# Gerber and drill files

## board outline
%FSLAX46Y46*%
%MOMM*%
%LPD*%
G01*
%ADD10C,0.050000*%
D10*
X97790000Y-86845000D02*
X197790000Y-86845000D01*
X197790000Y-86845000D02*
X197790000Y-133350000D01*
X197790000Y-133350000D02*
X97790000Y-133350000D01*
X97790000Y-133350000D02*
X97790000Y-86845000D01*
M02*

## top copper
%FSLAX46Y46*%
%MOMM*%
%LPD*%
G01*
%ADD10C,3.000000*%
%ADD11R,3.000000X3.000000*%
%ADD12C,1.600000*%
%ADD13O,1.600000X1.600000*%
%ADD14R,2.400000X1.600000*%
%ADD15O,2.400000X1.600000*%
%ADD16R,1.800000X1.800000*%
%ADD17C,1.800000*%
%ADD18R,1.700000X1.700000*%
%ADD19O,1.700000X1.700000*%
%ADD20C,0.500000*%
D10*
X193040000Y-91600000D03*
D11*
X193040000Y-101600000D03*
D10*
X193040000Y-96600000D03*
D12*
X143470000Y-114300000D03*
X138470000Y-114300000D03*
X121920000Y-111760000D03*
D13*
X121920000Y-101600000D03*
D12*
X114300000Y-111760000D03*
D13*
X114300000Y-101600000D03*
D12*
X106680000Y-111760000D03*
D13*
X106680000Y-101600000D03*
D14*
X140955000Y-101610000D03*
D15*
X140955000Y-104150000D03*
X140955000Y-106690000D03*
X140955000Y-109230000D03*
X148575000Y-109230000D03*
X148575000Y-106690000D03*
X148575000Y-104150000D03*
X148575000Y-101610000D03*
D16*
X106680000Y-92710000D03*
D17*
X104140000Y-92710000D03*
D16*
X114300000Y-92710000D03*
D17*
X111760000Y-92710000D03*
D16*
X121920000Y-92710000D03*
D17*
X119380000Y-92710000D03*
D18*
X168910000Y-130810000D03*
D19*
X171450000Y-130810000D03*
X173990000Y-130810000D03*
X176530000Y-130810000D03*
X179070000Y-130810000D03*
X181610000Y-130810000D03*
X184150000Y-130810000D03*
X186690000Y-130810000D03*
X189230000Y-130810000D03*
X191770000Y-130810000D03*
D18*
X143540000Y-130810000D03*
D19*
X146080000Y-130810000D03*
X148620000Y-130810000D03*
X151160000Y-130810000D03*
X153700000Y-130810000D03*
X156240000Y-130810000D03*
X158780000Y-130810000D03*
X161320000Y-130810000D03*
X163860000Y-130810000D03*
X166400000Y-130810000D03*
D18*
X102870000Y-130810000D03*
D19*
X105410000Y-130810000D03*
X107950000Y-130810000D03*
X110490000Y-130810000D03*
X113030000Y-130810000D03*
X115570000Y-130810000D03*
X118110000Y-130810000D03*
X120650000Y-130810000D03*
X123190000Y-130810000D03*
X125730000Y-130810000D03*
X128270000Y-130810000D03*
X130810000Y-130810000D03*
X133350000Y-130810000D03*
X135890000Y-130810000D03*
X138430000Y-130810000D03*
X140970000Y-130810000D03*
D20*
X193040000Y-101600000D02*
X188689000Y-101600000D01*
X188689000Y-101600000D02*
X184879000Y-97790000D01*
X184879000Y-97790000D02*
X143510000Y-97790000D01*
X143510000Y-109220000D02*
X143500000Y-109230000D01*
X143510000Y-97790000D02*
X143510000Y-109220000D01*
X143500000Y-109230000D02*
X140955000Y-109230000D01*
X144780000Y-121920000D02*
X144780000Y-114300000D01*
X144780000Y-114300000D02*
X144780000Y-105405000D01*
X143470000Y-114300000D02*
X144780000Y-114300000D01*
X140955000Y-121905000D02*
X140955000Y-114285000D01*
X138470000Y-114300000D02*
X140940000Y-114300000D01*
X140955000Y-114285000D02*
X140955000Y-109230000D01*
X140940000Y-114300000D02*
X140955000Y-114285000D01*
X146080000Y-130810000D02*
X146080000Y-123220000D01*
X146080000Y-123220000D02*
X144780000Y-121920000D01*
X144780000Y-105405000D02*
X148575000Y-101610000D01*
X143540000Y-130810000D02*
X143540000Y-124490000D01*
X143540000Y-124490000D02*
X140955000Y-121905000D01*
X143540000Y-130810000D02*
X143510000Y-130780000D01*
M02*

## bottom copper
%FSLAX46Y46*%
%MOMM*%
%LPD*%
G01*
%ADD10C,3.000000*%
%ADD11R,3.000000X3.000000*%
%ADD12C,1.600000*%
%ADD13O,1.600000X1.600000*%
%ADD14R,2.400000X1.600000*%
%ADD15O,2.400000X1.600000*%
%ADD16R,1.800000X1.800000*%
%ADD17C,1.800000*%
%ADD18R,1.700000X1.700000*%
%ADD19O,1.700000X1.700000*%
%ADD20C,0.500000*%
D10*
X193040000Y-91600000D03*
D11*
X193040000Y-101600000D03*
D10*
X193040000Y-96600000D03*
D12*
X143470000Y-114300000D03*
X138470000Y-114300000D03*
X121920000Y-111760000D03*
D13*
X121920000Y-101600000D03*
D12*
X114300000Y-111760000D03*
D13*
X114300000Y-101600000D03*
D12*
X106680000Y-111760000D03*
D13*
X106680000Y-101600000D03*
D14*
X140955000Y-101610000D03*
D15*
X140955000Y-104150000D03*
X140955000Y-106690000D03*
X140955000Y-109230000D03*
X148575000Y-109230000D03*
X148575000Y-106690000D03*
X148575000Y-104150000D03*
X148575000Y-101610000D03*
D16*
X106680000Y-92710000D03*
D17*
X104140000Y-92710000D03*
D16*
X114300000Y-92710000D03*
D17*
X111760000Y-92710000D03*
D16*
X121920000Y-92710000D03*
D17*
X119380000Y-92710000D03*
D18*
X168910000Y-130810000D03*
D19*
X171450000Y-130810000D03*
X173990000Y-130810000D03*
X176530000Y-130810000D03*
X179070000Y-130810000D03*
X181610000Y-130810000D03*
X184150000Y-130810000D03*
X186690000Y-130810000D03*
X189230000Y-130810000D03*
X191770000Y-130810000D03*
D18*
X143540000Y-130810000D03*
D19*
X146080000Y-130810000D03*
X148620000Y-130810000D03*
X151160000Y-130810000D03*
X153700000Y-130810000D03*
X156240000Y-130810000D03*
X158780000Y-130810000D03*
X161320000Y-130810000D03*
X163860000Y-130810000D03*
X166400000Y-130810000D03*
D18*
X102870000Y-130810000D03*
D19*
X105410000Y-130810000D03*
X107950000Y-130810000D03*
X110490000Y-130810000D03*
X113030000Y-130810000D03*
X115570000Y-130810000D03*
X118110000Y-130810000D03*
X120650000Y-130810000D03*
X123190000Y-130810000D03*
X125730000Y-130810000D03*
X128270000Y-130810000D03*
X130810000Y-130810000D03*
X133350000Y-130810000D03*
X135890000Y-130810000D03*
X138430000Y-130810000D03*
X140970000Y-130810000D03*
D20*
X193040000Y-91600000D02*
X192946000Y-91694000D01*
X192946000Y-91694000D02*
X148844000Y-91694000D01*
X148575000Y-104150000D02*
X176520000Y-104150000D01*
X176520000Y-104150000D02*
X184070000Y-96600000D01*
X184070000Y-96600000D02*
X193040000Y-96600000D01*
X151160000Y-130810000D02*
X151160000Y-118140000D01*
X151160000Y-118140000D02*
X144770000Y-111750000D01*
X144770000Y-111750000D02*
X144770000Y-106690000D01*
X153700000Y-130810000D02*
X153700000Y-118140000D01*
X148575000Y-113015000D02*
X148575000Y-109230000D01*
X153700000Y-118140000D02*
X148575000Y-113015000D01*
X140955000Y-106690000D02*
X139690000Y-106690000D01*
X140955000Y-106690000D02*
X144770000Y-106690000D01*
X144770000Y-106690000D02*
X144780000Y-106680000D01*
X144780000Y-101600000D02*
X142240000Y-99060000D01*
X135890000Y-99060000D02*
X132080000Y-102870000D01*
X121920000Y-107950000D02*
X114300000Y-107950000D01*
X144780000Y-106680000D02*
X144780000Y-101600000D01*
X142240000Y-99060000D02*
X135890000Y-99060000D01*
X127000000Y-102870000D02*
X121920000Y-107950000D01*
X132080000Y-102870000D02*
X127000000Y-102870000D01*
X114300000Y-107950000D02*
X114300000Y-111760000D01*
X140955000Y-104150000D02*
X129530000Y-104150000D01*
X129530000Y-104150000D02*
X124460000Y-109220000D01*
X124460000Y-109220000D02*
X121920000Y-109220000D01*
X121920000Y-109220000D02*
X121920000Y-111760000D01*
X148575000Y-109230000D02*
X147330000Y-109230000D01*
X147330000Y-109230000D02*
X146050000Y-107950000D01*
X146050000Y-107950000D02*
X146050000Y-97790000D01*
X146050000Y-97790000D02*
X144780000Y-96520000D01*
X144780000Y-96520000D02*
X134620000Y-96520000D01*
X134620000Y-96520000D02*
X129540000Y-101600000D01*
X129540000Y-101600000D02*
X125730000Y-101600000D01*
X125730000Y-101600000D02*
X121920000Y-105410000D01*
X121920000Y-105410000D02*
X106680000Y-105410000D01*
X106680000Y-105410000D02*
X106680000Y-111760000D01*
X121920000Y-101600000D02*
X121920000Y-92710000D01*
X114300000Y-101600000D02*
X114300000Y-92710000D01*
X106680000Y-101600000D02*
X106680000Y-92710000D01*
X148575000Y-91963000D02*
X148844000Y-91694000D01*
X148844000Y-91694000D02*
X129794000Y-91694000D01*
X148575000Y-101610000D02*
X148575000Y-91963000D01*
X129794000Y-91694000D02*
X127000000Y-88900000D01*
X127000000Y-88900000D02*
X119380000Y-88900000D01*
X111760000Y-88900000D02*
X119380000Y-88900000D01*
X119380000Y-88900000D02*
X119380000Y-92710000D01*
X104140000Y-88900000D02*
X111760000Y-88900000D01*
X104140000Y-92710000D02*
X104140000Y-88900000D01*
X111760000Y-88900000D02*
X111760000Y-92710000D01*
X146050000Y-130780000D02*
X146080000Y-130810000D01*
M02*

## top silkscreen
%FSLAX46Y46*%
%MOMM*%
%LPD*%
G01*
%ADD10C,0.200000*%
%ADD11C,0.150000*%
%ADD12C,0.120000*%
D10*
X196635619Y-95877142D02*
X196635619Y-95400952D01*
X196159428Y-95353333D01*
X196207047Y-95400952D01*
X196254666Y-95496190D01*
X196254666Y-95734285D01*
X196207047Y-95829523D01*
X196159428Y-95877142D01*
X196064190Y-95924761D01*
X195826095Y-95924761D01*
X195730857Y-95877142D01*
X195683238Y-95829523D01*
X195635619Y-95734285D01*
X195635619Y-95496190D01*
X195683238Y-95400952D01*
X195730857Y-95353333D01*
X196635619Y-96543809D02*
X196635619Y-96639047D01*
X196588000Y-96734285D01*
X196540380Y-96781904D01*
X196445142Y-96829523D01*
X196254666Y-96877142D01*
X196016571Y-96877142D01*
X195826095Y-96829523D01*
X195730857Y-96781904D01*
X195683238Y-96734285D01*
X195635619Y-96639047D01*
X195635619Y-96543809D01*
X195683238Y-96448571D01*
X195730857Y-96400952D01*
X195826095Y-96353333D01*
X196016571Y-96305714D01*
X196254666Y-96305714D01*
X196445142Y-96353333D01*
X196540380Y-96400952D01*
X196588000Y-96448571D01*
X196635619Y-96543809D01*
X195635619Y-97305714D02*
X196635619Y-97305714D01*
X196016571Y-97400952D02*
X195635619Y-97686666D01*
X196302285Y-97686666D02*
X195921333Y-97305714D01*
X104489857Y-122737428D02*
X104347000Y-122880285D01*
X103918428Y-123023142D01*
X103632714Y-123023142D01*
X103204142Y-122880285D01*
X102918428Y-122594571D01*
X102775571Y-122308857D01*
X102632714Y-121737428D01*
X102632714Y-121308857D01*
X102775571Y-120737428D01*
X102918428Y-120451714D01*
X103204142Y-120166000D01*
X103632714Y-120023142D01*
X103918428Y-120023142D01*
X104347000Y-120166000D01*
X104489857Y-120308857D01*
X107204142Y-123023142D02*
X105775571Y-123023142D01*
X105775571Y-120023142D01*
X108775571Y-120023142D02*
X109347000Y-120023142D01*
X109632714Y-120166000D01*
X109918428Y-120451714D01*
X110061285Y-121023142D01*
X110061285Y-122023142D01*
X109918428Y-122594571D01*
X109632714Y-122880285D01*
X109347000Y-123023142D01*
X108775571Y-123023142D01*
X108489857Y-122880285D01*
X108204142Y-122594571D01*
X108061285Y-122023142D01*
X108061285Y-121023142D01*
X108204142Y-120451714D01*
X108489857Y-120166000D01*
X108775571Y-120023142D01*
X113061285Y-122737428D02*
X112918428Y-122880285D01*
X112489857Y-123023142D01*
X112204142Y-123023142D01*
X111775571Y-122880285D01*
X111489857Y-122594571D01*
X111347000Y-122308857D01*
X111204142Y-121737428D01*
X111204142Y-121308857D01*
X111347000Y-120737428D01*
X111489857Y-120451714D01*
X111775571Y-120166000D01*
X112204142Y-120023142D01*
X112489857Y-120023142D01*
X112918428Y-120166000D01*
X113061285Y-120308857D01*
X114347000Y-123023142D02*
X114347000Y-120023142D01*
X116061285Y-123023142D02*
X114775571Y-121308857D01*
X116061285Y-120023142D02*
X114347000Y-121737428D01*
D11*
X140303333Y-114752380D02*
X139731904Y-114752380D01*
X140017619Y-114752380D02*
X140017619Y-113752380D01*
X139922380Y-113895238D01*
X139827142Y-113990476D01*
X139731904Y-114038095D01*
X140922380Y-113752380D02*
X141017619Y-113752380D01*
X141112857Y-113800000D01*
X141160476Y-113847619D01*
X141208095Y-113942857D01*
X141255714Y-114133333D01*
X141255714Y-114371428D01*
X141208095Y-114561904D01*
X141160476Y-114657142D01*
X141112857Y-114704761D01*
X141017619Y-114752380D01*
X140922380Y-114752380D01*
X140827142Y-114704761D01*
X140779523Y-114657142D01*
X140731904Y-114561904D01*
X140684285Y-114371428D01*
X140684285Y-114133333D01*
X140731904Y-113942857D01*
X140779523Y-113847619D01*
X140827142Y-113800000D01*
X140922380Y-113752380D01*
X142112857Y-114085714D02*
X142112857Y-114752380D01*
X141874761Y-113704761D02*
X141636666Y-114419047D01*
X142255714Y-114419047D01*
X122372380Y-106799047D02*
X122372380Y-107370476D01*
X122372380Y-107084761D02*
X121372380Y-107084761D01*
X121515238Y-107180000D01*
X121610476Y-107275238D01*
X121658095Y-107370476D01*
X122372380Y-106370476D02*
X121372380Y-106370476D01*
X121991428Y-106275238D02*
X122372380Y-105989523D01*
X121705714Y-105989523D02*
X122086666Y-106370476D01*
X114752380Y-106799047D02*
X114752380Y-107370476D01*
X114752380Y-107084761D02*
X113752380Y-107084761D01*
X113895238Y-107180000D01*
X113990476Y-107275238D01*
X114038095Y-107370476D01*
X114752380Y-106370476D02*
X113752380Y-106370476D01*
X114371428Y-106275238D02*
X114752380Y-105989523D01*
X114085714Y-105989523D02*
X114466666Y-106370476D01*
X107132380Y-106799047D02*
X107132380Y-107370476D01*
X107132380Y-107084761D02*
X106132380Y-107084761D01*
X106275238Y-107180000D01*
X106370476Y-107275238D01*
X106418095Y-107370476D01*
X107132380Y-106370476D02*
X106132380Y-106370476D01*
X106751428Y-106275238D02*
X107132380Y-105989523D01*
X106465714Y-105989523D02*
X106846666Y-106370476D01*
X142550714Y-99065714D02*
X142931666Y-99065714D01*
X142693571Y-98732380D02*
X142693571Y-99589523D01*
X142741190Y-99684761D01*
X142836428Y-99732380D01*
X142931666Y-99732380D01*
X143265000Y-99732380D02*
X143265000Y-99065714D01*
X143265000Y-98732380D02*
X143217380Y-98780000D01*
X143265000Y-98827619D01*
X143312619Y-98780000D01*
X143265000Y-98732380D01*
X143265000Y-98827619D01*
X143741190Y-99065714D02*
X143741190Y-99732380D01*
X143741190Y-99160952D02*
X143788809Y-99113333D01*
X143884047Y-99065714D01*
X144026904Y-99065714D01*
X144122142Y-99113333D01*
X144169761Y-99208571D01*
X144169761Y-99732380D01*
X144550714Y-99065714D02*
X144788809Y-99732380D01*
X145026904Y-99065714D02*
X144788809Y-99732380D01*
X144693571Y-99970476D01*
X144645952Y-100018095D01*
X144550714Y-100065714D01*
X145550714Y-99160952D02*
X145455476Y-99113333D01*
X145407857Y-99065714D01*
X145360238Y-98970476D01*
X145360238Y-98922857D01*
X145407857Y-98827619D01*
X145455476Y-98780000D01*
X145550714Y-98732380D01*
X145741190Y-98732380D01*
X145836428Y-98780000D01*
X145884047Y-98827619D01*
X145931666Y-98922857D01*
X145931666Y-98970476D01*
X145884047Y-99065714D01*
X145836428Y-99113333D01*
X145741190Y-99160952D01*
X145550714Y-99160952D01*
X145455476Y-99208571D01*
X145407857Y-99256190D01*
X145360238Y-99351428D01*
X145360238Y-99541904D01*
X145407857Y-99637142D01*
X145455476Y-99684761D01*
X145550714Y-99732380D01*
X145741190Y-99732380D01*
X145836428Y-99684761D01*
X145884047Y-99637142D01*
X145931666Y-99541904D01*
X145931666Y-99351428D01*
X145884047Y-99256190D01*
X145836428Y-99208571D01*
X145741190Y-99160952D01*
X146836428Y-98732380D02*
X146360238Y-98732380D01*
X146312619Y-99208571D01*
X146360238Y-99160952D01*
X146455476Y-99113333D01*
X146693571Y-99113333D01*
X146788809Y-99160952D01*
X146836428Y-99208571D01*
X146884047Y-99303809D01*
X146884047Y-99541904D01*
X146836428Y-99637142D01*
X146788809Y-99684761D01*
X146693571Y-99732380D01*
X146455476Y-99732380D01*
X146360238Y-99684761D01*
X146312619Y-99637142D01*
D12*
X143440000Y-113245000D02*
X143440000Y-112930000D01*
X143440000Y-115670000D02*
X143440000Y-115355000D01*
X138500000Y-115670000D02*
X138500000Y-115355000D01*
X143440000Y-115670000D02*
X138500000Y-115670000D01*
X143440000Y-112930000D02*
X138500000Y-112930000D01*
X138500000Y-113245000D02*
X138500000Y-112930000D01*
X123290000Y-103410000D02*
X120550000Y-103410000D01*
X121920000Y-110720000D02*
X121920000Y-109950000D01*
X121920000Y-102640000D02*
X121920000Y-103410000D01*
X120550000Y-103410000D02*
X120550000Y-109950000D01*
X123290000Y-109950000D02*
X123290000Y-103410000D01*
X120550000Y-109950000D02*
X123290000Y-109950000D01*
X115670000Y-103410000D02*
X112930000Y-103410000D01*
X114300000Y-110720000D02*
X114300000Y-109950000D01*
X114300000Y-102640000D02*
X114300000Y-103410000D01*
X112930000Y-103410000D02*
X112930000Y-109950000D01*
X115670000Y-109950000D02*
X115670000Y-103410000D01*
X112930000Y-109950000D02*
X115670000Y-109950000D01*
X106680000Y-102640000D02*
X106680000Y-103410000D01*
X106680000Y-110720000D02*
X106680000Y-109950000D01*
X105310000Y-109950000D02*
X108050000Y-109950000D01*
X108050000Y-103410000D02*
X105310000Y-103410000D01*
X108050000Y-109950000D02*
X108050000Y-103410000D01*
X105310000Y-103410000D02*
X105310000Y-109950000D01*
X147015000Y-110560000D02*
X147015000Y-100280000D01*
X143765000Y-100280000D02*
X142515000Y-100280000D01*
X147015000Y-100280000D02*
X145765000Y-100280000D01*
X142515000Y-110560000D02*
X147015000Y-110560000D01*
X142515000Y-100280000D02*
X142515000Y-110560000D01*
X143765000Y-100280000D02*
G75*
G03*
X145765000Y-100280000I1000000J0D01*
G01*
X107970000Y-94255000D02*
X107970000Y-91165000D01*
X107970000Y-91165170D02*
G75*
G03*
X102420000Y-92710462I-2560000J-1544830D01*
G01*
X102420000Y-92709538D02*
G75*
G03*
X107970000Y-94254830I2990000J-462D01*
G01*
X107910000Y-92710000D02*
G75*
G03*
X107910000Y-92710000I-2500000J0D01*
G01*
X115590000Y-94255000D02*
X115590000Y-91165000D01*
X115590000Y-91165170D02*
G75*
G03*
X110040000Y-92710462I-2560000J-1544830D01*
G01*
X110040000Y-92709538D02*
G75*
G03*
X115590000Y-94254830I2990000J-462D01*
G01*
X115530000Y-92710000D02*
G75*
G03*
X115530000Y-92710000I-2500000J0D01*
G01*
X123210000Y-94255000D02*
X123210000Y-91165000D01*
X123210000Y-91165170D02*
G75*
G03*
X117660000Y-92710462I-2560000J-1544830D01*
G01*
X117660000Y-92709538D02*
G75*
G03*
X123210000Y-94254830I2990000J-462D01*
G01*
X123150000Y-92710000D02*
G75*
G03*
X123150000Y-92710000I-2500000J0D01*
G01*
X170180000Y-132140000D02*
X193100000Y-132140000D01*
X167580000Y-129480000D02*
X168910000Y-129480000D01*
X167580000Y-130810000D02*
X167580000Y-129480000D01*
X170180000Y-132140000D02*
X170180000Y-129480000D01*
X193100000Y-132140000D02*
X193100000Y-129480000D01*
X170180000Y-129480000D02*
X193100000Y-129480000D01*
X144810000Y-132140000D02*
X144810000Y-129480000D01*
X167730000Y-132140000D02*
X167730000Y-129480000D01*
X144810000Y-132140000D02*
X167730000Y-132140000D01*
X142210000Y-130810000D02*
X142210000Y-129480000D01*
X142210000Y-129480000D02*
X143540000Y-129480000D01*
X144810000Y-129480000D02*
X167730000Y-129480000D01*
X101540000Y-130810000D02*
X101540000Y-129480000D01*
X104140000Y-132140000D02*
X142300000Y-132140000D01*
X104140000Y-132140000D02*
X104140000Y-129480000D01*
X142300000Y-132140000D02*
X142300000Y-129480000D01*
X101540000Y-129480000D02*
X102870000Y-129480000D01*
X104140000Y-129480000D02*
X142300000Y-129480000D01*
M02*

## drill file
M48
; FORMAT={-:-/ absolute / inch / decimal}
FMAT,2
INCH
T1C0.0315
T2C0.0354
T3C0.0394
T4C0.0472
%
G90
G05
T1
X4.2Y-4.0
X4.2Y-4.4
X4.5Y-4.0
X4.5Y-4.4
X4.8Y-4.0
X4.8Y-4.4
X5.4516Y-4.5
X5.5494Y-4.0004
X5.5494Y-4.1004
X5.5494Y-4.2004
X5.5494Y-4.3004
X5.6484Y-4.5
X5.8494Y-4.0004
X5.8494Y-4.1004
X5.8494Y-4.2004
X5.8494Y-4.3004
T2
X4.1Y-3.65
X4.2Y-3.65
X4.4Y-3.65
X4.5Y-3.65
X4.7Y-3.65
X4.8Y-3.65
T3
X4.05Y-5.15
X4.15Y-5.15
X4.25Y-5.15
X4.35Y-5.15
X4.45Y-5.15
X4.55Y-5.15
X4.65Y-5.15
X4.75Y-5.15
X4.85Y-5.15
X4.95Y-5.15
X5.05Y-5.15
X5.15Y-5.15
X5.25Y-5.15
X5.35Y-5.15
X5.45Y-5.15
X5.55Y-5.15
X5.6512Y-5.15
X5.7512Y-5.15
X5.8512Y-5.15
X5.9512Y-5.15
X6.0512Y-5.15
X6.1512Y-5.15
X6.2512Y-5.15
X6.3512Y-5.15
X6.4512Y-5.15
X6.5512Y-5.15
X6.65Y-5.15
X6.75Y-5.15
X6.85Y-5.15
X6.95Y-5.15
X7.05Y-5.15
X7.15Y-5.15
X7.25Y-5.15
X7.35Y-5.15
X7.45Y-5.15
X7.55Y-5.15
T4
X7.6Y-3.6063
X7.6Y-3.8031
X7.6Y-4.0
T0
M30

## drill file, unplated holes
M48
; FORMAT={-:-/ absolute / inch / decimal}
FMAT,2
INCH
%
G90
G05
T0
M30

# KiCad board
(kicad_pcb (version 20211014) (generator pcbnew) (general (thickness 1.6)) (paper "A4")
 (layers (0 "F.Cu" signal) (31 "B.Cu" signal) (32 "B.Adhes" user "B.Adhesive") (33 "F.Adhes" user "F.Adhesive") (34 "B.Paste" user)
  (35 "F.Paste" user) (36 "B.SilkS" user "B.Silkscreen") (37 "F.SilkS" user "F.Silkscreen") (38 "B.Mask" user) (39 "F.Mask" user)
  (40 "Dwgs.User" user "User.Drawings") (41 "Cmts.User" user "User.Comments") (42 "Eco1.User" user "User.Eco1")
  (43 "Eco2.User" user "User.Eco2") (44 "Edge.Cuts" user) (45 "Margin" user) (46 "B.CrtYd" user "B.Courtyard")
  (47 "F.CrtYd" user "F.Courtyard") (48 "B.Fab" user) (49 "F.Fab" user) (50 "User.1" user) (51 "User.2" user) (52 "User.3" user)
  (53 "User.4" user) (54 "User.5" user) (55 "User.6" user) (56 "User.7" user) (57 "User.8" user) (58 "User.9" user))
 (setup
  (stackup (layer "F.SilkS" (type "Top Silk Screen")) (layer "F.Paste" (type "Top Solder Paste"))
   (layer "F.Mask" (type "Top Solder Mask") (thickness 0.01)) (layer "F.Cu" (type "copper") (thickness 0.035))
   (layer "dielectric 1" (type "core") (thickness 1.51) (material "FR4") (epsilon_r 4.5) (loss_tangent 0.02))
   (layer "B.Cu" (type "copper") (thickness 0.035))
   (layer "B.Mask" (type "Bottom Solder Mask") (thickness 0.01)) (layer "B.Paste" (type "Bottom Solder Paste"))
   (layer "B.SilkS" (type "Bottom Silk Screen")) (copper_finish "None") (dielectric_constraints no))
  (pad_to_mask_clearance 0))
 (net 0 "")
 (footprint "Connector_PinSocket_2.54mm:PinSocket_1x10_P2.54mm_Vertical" (layer "F.Cu") (at 168.91 130.81 90)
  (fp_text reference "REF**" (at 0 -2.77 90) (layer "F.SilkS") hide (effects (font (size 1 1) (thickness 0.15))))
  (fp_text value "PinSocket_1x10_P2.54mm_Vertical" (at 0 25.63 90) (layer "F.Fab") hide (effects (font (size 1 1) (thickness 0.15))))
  (fp_line (start -1.33 1.27) (end -1.33 24.19) (layer "F.SilkS") (width 0.12))
  (fp_line (start 1.33 -1.33) (end 1.33 0) (layer "F.SilkS") (width 0.12))
  (fp_line (start 0 -1.33) (end 1.33 -1.33) (layer "F.SilkS") (width 0.12))
  (fp_line (start -1.33 1.27) (end 1.33 1.27) (layer "F.SilkS") (width 0.12))
  (fp_line (start -1.33 24.19) (end 1.33 24.19) (layer "F.SilkS") (width 0.12))
  (fp_line (start 1.33 1.27) (end 1.33 24.19) (layer "F.SilkS") (width 0.12))
  (pad "1" thru_hole rect (at 0 0 90) (size 1.7 1.7) (drill 1) (layers F&B.Cu *.Mask))
  (pad "2" thru_hole oval (at 0 2.54 90) (size 1.7 1.7) (drill 1) (layers F&B.Cu *.Mask))
  (pad "3" thru_hole oval (at 0 5.08 90) (size 1.7 1.7) (drill 1) (layers F&B.Cu *.Mask))
  (pad "4" thru_hole oval (at 0 7.62 90) (size 1.7 1.7) (drill 1) (layers F&B.Cu *.Mask))
  (pad "5" thru_hole oval (at 0 10.16 90) (size 1.7 1.7) (drill 1) (layers F&B.Cu *.Mask))
  (pad "6" thru_hole oval (at 0 12.7 90) (size 1.7 1.7) (drill 1) (layers F&B.Cu *.Mask))
  (pad "7" thru_hole oval (at 0 15.24 90) (size 1.7 1.7) (drill 1) (layers F&B.Cu *.Mask))
  (pad "8" thru_hole oval (at 0 17.78 90) (size 1.7 1.7) (drill 1) (layers F&B.Cu *.Mask))
  (pad "9" thru_hole oval (at 0 20.32 90) (size 1.7 1.7) (drill 1) (layers F&B.Cu *.Mask))
  (pad "10" thru_hole oval (at 0 22.86 90) (size 1.7 1.7) (drill 1) (layers F&B.Cu *.Mask)))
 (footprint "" (layer "F.Cu") (at 193.04 96.6 -90)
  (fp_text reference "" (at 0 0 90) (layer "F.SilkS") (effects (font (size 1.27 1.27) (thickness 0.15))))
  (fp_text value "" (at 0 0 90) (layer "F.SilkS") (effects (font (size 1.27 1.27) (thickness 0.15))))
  (pad "2" thru_hole circle (at 0 0) (size 3 3) (drill 1.2) (layers F&B.Cu *.Mask)))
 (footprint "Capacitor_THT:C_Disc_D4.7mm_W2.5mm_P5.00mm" (layer "F.Cu") (at 143.47 114.3 180)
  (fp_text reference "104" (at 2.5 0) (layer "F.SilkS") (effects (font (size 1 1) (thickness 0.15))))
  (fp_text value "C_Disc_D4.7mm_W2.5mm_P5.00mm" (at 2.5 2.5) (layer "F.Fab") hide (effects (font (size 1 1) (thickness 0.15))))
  (fp_line (start 0.03 1.055) (end 0.03 1.37) (layer "F.SilkS") (width 0.12))
  (fp_line (start 0.03 -1.37) (end 0.03 -1.055) (layer "F.SilkS") (width 0.12))
  (fp_line (start 4.97 -1.37) (end 4.97 -1.055) (layer "F.SilkS") (width 0.12))
  (fp_line (start 0.03 -1.37) (end 4.97 -1.37) (layer "F.SilkS") (width 0.12))
  (fp_line (start 0.03 1.37) (end 4.97 1.37) (layer "F.SilkS") (width 0.12))
  (fp_line (start 4.97 1.055) (end 4.97 1.37) (layer "F.SilkS") (width 0.12))
  (pad "1" thru_hole circle (at 0 0 180) (size 1.6 1.6) (drill 0.8) (layers F&B.Cu *.Mask))
  (pad "2" thru_hole circle (at 5 0 180) (size 1.6 1.6) (drill 0.8) (layers F&B.Cu *.Mask)))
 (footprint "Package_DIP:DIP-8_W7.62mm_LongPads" (layer "F.Cu") (at 140.955 101.61)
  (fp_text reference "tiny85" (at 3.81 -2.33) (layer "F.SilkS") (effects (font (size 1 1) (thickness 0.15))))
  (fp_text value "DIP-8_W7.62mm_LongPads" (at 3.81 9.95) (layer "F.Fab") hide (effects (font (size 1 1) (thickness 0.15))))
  (fp_line (start 6.06 8.95) (end 6.06 -1.33) (layer "F.SilkS") (width 0.12))
  (fp_line (start 2.81 -1.33) (end 1.56 -1.33) (layer "F.SilkS") (width 0.12))
  (fp_line (start 6.06 -1.33) (end 4.81 -1.33) (layer "F.SilkS") (width 0.12))
  (fp_line (start 1.56 8.95) (end 6.06 8.95) (layer "F.SilkS") (width 0.12))
  (fp_line (start 1.56 -1.33) (end 1.56 8.95) (layer "F.SilkS") (width 0.12))
  (fp_arc (start 4.81 -1.33) (mid 3.81 -0.33) (end 2.81 -1.33) (layer "F.SilkS") (width 0.12))
  (pad "1" thru_hole rect (at 0 0) (size 2.4 1.6) (drill 0.8) (layers F&B.Cu *.Mask))
  (pad "2" thru_hole oval (at 0 2.54) (size 2.4 1.6) (drill 0.8) (layers F&B.Cu *.Mask))
  (pad "3" thru_hole oval (at 0 5.08) (size 2.4 1.6) (drill 0.8) (layers F&B.Cu *.Mask))
  (pad "4" thru_hole oval (at 0 7.62) (size 2.4 1.6) (drill 0.8) (layers F&B.Cu *.Mask))
  (pad "5" thru_hole oval (at 7.62 7.62) (size 2.4 1.6) (drill 0.8) (layers F&B.Cu *.Mask))
  (pad "6" thru_hole oval (at 7.62 5.08) (size 2.4 1.6) (drill 0.8) (layers F&B.Cu *.Mask))
  (pad "7" thru_hole oval (at 7.62 2.54) (size 2.4 1.6) (drill 0.8) (layers F&B.Cu *.Mask))
  (pad "8" thru_hole oval (at 7.62 0) (size 2.4 1.6) (drill 0.8) (layers F&B.Cu *.Mask)))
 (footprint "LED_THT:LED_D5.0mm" (layer "F.Cu") (at 114.3 92.71 180)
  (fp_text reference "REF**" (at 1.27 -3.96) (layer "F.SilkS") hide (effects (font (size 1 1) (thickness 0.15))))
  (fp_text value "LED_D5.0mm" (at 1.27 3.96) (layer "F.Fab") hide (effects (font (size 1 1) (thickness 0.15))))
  (fp_line (start -1.29 -1.545) (end -1.29 1.545) (layer "F.SilkS") (width 0.12))
  (fp_arc (start 4.26 -0.000462) (mid 2.072002 2.880433) (end -1.29 1.54483) (layer "F.SilkS") (width 0.12))
  (fp_arc (start -1.29 -1.54483) (mid 2.072002 -2.880433) (end 4.26 0.000462) (layer "F.SilkS") (width 0.12))
  (fp_circle (center 1.27 0) (end 3.77 0) (layer "F.SilkS") (width 0.12) (fill none))
  (pad "1" thru_hole rect (at 0 0 180) (size 1.8 1.8) (drill 0.9) (layers F&B.Cu *.Mask))
  (pad "2" thru_hole circle (at 2.54 0 180) (size 1.8 1.8) (drill 0.9) (layers F&B.Cu *.Mask)))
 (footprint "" (layer "F.Cu") (at 193.04 91.6 -90)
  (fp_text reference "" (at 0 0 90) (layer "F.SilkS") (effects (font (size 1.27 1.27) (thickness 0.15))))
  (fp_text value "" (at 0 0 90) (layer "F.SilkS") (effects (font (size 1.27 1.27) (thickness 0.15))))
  (pad "3" thru_hole circle (at 0 0) (size 3 3) (drill 1.2) (layers F&B.Cu *.Mask)))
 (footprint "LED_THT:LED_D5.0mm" (layer "F.Cu") (at 121.92 92.71 180)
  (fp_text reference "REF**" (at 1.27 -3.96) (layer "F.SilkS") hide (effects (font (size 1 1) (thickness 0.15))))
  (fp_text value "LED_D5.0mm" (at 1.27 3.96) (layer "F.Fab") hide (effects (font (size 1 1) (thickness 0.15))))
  (fp_line (start -1.29 -1.545) (end -1.29 1.545) (layer "F.SilkS") (width 0.12))
  (fp_arc (start 4.26 -0.000462) (mid 2.072002 2.880433) (end -1.29 1.54483) (layer "F.SilkS") (width 0.12))
  (fp_arc (start -1.29 -1.54483) (mid 2.072002 -2.880433) (end 4.26 0.000462) (layer "F.SilkS") (width 0.12))
  (fp_circle (center 1.27 0) (end 3.77 0) (layer "F.SilkS") (width 0.12) (fill none))
  (pad "1" thru_hole rect (at 0 0 180) (size 1.8 1.8) (drill 0.9) (layers F&B.Cu *.Mask))
  (pad "2" thru_hole circle (at 2.54 0 180) (size 1.8 1.8) (drill 0.9) (layers F&B.Cu *.Mask)))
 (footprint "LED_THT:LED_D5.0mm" (layer "F.Cu") (at 106.68 92.71 180)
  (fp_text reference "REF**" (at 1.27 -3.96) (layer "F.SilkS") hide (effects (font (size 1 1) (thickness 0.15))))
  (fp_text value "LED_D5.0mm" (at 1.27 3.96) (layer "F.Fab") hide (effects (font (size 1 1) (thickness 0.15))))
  (fp_line (start -1.29 -1.545) (end -1.29 1.545) (layer "F.SilkS") (width 0.12))
  (fp_arc (start 4.26 -0.000462) (mid 2.072002 2.880433) (end -1.29 1.54483) (layer "F.SilkS") (width 0.12))
  (fp_arc (start -1.29 -1.54483) (mid 2.072002 -2.880433) (end 4.26 0.000462) (layer "F.SilkS") (width 0.12))
  (fp_circle (center 1.27 0) (end 3.77 0) (layer "F.SilkS") (width 0.12) (fill none))
  (pad "1" thru_hole rect (at 0 0 180) (size 1.8 1.8) (drill 0.9) (layers F&B.Cu *.Mask))
  (pad "2" thru_hole circle (at 2.54 0 180) (size 1.8 1.8) (drill 0.9) (layers F&B.Cu *.Mask)))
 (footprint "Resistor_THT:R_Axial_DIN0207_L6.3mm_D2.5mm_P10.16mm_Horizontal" (layer "F.Cu") (at 121.92 111.76 90)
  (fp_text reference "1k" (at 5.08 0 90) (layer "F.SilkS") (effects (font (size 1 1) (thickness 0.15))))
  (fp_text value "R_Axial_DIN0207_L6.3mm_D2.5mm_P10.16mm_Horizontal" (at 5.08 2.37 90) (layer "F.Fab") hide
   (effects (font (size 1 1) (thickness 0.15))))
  (fp_line (start 8.35 1.37) (end 8.35 -1.37) (layer "F.SilkS") (width 0.12))
  (fp_line (start 1.04 0) (end 1.81 0) (layer "F.SilkS") (width 0.12))
  (fp_line (start 9.12 0) (end 8.35 0) (layer "F.SilkS") (width 0.12))
  (fp_line (start 8.35 -1.37) (end 1.81 -1.37) (layer "F.SilkS") (width 0.12))
  (fp_line (start 1.81 1.37) (end 8.35 1.37) (layer "F.SilkS") (width 0.12))
  (fp_line (start 1.81 -1.37) (end 1.81 1.37) (layer "F.SilkS") (width 0.12))
  (pad "1" thru_hole circle (at 0 0 90) (size 1.6 1.6) (drill 0.8) (layers F&B.Cu *.Mask))
  (pad "2" thru_hole oval (at 10.16 0 90) (size 1.6 1.6) (drill 0.8) (layers F&B.Cu *.Mask)))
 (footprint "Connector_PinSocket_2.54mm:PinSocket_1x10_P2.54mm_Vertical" (layer "F.Cu") (at 143.54 130.81 90)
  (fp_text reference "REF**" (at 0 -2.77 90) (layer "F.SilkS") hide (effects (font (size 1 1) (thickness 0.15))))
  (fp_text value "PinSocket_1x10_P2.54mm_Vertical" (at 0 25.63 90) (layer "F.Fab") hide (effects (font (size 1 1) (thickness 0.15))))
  (fp_line (start -1.33 1.27) (end 1.33 1.27) (layer "F.SilkS") (width 0.12))
  (fp_line (start -1.33 24.19) (end 1.33 24.19) (layer "F.SilkS") (width 0.12))
  (fp_line (start -1.33 1.27) (end -1.33 24.19) (layer "F.SilkS") (width 0.12))
  (fp_line (start 0 -1.33) (end 1.33 -1.33) (layer "F.SilkS") (width 0.12))
  (fp_line (start 1.33 -1.33) (end 1.33 0) (layer "F.SilkS") (width 0.12))
  (fp_line (start 1.33 1.27) (end 1.33 24.19) (layer "F.SilkS") (width 0.12))
  (pad "1" thru_hole rect (at 0 0 90) (size 1.7 1.7) (drill 1) (layers F&B.Cu *.Mask))
  (pad "2" thru_hole oval (at 0 2.54 90) (size 1.7 1.7) (drill 1) (layers F&B.Cu *.Mask))
  (pad "3" thru_hole oval (at 0 5.08 90) (size 1.7 1.7) (drill 1) (layers F&B.Cu *.Mask))
  (pad "4" thru_hole oval (at 0 7.62 90) (size 1.7 1.7) (drill 1) (layers F&B.Cu *.Mask))
  (pad "5" thru_hole oval (at 0 10.16 90) (size 1.7 1.7) (drill 1) (layers F&B.Cu *.Mask))
  (pad "6" thru_hole oval (at 0 12.7 90) (size 1.7 1.7) (drill 1) (layers F&B.Cu *.Mask))
  (pad "7" thru_hole oval (at 0 15.24 90) (size 1.7 1.7) (drill 1) (layers F&B.Cu *.Mask))
  (pad "8" thru_hole oval (at 0 17.78 90) (size 1.7 1.7) (drill 1) (layers F&B.Cu *.Mask))
  (pad "9" thru_hole oval (at 0 20.32 90) (size 1.7 1.7) (drill 1) (layers F&B.Cu *.Mask))
  (pad "10" thru_hole oval (at 0 22.86 90) (size 1.7 1.7) (drill 1) (layers F&B.Cu *.Mask)))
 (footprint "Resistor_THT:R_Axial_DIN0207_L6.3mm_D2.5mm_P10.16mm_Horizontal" (layer "F.Cu") (at 106.68 111.76 90)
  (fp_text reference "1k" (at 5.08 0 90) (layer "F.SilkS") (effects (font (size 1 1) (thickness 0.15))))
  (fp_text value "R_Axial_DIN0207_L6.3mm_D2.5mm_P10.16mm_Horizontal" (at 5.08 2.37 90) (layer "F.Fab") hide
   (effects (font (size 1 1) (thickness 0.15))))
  (fp_line (start 8.35 1.37) (end 8.35 -1.37) (layer "F.SilkS") (width 0.12))
  (fp_line (start 1.04 0) (end 1.81 0) (layer "F.SilkS") (width 0.12))
  (fp_line (start 9.12 0) (end 8.35 0) (layer "F.SilkS") (width 0.12))
  (fp_line (start 8.35 -1.37) (end 1.81 -1.37) (layer "F.SilkS") (width 0.12))
  (fp_line (start 1.81 1.37) (end 8.35 1.37) (layer "F.SilkS") (width 0.12))
  (fp_line (start 1.81 -1.37) (end 1.81 1.37) (layer "F.SilkS") (width 0.12))
  (pad "1" thru_hole circle (at 0 0 90) (size 1.6 1.6) (drill 0.8) (layers *.Cu *.Mask))
  (pad "2" thru_hole oval (at 10.16 0 90) (size 1.6 1.6) (drill 0.8) (layers *.Cu *.Mask)))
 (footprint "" (layer "F.Cu") (at 193.04 101.6 -90)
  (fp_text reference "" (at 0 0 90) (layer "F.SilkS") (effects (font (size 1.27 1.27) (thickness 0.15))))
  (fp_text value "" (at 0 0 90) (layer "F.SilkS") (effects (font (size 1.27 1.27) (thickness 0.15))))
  (pad "1" thru_hole rect (at 0 0) (size 3 3) (drill 1.2) (layers F&B.Cu *.Mask)))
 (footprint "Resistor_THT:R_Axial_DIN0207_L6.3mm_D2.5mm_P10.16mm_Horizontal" (layer "F.Cu") (at 114.3 111.76 90)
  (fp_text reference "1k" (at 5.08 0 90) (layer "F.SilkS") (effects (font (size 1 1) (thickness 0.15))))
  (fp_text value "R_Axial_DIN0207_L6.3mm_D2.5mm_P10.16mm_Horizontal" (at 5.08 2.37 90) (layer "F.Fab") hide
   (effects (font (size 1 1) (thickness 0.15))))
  (fp_line (start 8.35 1.37) (end 8.35 -1.37) (layer "F.SilkS") (width 0.12))
  (fp_line (start 1.04 0) (end 1.81 0) (layer "F.SilkS") (width 0.12))
  (fp_line (start 9.12 0) (end 8.35 0) (layer "F.SilkS") (width 0.12))
  (fp_line (start 8.35 -1.37) (end 1.81 -1.37) (layer "F.SilkS") (width 0.12))
  (fp_line (start 1.81 1.37) (end 8.35 1.37) (layer "F.SilkS") (width 0.12))
  (fp_line (start 1.81 -1.37) (end 1.81 1.37) (layer "F.SilkS") (width 0.12))
  (pad "1" thru_hole circle (at 0 0 90) (size 1.6 1.6) (drill 0.8) (layers F&B.Cu *.Mask))
  (pad "2" thru_hole oval (at 10.16 0 90) (size 1.6 1.6) (drill 0.8) (layers F&B.Cu *.Mask)))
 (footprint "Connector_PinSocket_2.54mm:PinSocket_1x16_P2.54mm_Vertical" (layer "F.Cu") (at 102.87 130.81 90)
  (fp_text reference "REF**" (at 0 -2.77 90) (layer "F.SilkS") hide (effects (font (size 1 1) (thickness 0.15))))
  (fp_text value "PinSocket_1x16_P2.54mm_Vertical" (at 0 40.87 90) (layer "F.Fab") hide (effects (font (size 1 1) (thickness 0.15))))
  (fp_line (start 0 -1.33) (end 1.33 -1.33) (layer "F.SilkS") (width 0.12))
  (fp_line (start -1.33 1.27) (end -1.33 39.43) (layer "F.SilkS") (width 0.12))
  (fp_line (start -1.33 1.27) (end 1.33 1.27) (layer "F.SilkS") (width 0.12))
  (fp_line (start -1.33 39.43) (end 1.33 39.43) (layer "F.SilkS") (width 0.12))
  (fp_line (start 1.33 -1.33) (end 1.33 0) (layer "F.SilkS") (width 0.12))
  (fp_line (start 1.33 1.27) (end 1.33 39.43) (layer "F.SilkS") (width 0.12))
  (pad "1" thru_hole rect (at 0 0 90) (size 1.7 1.7) (drill 1) (layers F&B.Cu *.Mask))
  (pad "2" thru_hole oval (at 0 2.54 90) (size 1.7 1.7) (drill 1) (layers F&B.Cu *.Mask))
  (pad "3" thru_hole oval (at 0 5.08 90) (size 1.7 1.7) (drill 1) (layers F&B.Cu *.Mask))
  (pad "4" thru_hole oval (at 0 7.62 90) (size 1.7 1.7) (drill 1) (layers F&B.Cu *.Mask))
  (pad "5" thru_hole oval (at 0 10.16 90) (size 1.7 1.7) (drill 1) (layers F&B.Cu *.Mask))
  (pad "6" thru_hole oval (at 0 12.7 90) (size 1.7 1.7) (drill 1) (layers F&B.Cu *.Mask))
  (pad "7" thru_hole oval (at 0 15.24 90) (size 1.7 1.7) (drill 1) (layers F&B.Cu *.Mask))
  (pad "8" thru_hole oval (at 0 17.78 90) (size 1.7 1.7) (drill 1) (layers F&B.Cu *.Mask))
  (pad "9" thru_hole oval (at 0 20.32 90) (size 1.7 1.7) (drill 1) (layers F&B.Cu *.Mask))
  (pad "10" thru_hole oval (at 0 22.86 90) (size 1.7 1.7) (drill 1) (layers F&B.Cu *.Mask))
  (pad "11" thru_hole oval (at 0 25.4 90) (size 1.7 1.7) (drill 1) (layers F&B.Cu *.Mask))
  (pad "12" thru_hole oval (at 0 27.94 90) (size 1.7 1.7) (drill 1) (layers F&B.Cu *.Mask))
  (pad "13" thru_hole oval (at 0 30.48 90) (size 1.7 1.7) (drill 1) (layers F&B.Cu *.Mask))
  (pad "14" thru_hole oval (at 0 33.02 90) (size 1.7 1.7) (drill 1) (layers F&B.Cu *.Mask))
  (pad "15" thru_hole oval (at 0 35.56 90) (size 1.7 1.7) (drill 1) (layers F&B.Cu *.Mask))
  (pad "16" thru_hole oval (at 0 38.1 90) (size 1.7 1.7) (drill 1) (layers F&B.Cu *.Mask)))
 (gr_rect (start 97.79 86.845) (end 197.79 133.35) (layer "Edge.Cuts") (width 0.05) (fill none))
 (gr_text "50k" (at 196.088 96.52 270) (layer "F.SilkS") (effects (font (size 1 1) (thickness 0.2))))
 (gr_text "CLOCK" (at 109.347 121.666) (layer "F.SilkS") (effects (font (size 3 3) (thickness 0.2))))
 (segment (start 143.47 114.3) (end 144.78 114.3) (width 0.5) (layer "F.Cu") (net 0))
 (segment (start 144.78 121.92) (end 144.78 114.3) (width 0.5) (layer "F.Cu") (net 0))
 (segment (start 184.879 97.79) (end 143.51 97.79) (width 0.5) (layer "F.Cu") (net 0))
 (segment (start 143.5 109.23) (end 140.955 109.23) (width 0.5) (layer "F.Cu") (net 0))
 (segment (start 193.04 101.6) (end 188.689 101.6) (width 0.5) (layer "F.Cu") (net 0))
 (segment (start 146.08 123.22) (end 144.78 121.92) (width 0.5) (layer "F.Cu") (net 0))
 (segment (start 144.78 114.3) (end 144.78 105.405) (width 0.5) (layer "F.Cu") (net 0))
 (segment (start 140.955 121.905) (end 140.955 114.285) (width 0.5) (layer "F.Cu") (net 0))
 (segment (start 143.51 109.22) (end 143.5 109.23) (width 0.5) (layer "F.Cu") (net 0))
 (segment (start 146.08 130.81) (end 146.08 123.22) (width 0.5) (layer "F.Cu") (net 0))
 (segment (start 143.51 97.79) (end 143.51 109.22) (width 0.5) (layer "F.Cu") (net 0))
 (segment (start 188.689 101.6) (end 184.879 97.79) (width 0.5) (layer "F.Cu") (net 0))
 (segment (start 143.54 130.81) (end 143.54 124.49) (width 0.5) (layer "F.Cu") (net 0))
 (segment (start 138.47 114.3) (end 140.94 114.3) (width 0.5) (layer "F.Cu") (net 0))
 (segment (start 140.955 114.285) (end 140.955 109.23) (width 0.5) (layer "F.Cu") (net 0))
 (segment (start 143.54 130.81) (end 143.51 130.78) (width 0.5) (layer "F.Cu") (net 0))
 (segment (start 144.78 105.405) (end 148.575 101.61) (width 0.5) (layer "F.Cu") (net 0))
 (segment (start 143.54 124.49) (end 140.955 121.905) (width 0.5) (layer "F.Cu") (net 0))
 (segment (start 140.94 114.3) (end 140.955 114.285) (width 0.5) (layer "F.Cu") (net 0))
 (segment (start 104.14 92.71) (end 104.14 88.9) (width 0.5) (layer "B.Cu") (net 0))
 (segment (start 140.955 104.15) (end 129.53 104.15) (width 0.5) (layer "B.Cu") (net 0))
 (segment (start 106.68 101.6) (end 106.68 92.71) (width 0.5) (layer "B.Cu") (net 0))
 (segment (start 193.04 91.6) (end 192.946 91.694) (width 0.5) (layer "B.Cu") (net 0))
 (segment (start 129.54 101.6) (end 125.73 101.6) (width 0.5) (layer "B.Cu") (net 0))
 (segment (start 146.05 130.78) (end 146.08 130.81) (width 0.5) (layer "B.Cu") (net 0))
 (segment (start 114.3 101.6) (end 114.3 92.71) (width 0.5) (layer "B.Cu") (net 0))
 (segment (start 146.05 107.95) (end 146.05 97.79) (width 0.5) (layer "B.Cu") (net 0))
 (segment (start 129.53 104.15) (end 124.46 109.22) (width 0.5) (layer "B.Cu") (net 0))
 (segment (start 148.844 91.694) (end 129.794 91.694) (width 0.5) (layer "B.Cu") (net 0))
 (segment (start 144.78 96.52) (end 134.62 96.52) (width 0.5) (layer "B.Cu") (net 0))
 (segment (start 119.38 88.9) (end 119.38 92.71) (width 0.5) (layer "B.Cu") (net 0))
 (segment (start 192.946 91.694) (end 148.844 91.694) (width 0.5) (layer "B.Cu") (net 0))
 (segment (start 132.08 102.87) (end 127 102.87) (width 0.5) (layer "B.Cu") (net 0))
 (segment (start 146.05 97.79) (end 144.78 96.52) (width 0.5) (layer "B.Cu") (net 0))
 (segment (start 148.575 109.23) (end 147.33 109.23) (width 0.5) (layer "B.Cu") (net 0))
 (segment (start 124.46 109.22) (end 121.92 109.22) (width 0.5) (layer "B.Cu") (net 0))
 (segment (start 127 88.9) (end 119.38 88.9) (width 0.5) (layer "B.Cu") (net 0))
 (segment (start 153.7 130.81) (end 153.7 118.14) (width 0.5) (layer "B.Cu") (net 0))
 (segment (start 148.575 104.15) (end 176.52 104.15) (width 0.5) (layer "B.Cu") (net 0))
 (segment (start 104.14 88.9) (end 111.76 88.9) (width 0.5) (layer "B.Cu") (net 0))
 (segment (start 121.92 109.22) (end 121.92 111.76) (width 0.5) (layer "B.Cu") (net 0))
 (segment (start 151.16 118.14) (end 144.77 111.75) (width 0.5) (layer "B.Cu") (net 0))
 (segment (start 148.575 113.015) (end 148.575 109.23) (width 0.5) (layer "B.Cu") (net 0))
 (segment (start 106.68 105.41) (end 106.68 111.76) (width 0.5) (layer "B.Cu") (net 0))
 (segment (start 184.07 96.6) (end 193.04 96.6) (width 0.5) (layer "B.Cu") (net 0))
 (segment (start 147.33 109.23) (end 146.05 107.95) (width 0.5) (layer "B.Cu") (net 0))
 (segment (start 127 102.87) (end 121.92 107.95) (width 0.5) (layer "B.Cu") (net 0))
 (segment (start 121.92 107.95) (end 114.3 107.95) (width 0.5) (layer "B.Cu") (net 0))
 (segment (start 135.89 99.06) (end 132.08 102.87) (width 0.5) (layer "B.Cu") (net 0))
 (segment (start 144.78 101.6) (end 142.24 99.06) (width 0.5) (layer "B.Cu") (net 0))
 (segment (start 129.794 91.694) (end 127 88.9) (width 0.5) (layer "B.Cu") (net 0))
 (segment (start 111.76 88.9) (end 111.76 92.71) (width 0.5) (layer "B.Cu") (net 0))
 (segment (start 148.575 101.61) (end 148.575 91.963) (width 0.5) (layer "B.Cu") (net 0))
 (segment (start 176.52 104.15) (end 184.07 96.6) (width 0.5) (layer "B.Cu") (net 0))
 (segment (start 151.16 130.81) (end 151.16 118.14) (width 0.5) (layer "B.Cu") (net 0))
 (segment (start 114.3 107.95) (end 114.3 111.76) (width 0.5) (layer "B.Cu") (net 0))
 (segment (start 140.955 106.69) (end 139.69 106.69) (width 0.5) (layer "B.Cu") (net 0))
 (segment (start 134.62 96.52) (end 129.54 101.6) (width 0.5) (layer "B.Cu") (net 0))
 (segment (start 144.77 106.69) (end 144.78 106.68) (width 0.5) (layer "B.Cu") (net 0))
 (segment (start 148.575 91.963) (end 148.844 91.694) (width 0.5) (layer "B.Cu") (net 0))
 (segment (start 144.78 106.68) (end 144.78 101.6) (width 0.5) (layer "B.Cu") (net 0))
 (segment (start 111.76 88.9) (end 119.38 88.9) (width 0.5) (layer "B.Cu") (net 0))
 (segment (start 140.955 106.69) (end 144.77 106.69) (width 0.5) (layer "B.Cu") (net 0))
 (segment (start 153.7 118.14) (end 148.575 113.015) (width 0.5) (layer "B.Cu") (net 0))
 (segment (start 125.73 101.6) (end 121.92 105.41) (width 0.5) (layer "B.Cu") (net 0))
 (segment (start 121.92 105.41) (end 106.68 105.41) (width 0.5) (layer "B.Cu") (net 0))
 (segment (start 144.77 111.75) (end 144.77 106.69) (width 0.5) (layer "B.Cu") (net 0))
 (segment (start 142.24 99.06) (end 135.89 99.06) (width 0.5) (layer "B.Cu") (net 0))
 (segment (start 121.92 101.6) (end 121.92 92.71) (width 0.5) (layer "B.Cu") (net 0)))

